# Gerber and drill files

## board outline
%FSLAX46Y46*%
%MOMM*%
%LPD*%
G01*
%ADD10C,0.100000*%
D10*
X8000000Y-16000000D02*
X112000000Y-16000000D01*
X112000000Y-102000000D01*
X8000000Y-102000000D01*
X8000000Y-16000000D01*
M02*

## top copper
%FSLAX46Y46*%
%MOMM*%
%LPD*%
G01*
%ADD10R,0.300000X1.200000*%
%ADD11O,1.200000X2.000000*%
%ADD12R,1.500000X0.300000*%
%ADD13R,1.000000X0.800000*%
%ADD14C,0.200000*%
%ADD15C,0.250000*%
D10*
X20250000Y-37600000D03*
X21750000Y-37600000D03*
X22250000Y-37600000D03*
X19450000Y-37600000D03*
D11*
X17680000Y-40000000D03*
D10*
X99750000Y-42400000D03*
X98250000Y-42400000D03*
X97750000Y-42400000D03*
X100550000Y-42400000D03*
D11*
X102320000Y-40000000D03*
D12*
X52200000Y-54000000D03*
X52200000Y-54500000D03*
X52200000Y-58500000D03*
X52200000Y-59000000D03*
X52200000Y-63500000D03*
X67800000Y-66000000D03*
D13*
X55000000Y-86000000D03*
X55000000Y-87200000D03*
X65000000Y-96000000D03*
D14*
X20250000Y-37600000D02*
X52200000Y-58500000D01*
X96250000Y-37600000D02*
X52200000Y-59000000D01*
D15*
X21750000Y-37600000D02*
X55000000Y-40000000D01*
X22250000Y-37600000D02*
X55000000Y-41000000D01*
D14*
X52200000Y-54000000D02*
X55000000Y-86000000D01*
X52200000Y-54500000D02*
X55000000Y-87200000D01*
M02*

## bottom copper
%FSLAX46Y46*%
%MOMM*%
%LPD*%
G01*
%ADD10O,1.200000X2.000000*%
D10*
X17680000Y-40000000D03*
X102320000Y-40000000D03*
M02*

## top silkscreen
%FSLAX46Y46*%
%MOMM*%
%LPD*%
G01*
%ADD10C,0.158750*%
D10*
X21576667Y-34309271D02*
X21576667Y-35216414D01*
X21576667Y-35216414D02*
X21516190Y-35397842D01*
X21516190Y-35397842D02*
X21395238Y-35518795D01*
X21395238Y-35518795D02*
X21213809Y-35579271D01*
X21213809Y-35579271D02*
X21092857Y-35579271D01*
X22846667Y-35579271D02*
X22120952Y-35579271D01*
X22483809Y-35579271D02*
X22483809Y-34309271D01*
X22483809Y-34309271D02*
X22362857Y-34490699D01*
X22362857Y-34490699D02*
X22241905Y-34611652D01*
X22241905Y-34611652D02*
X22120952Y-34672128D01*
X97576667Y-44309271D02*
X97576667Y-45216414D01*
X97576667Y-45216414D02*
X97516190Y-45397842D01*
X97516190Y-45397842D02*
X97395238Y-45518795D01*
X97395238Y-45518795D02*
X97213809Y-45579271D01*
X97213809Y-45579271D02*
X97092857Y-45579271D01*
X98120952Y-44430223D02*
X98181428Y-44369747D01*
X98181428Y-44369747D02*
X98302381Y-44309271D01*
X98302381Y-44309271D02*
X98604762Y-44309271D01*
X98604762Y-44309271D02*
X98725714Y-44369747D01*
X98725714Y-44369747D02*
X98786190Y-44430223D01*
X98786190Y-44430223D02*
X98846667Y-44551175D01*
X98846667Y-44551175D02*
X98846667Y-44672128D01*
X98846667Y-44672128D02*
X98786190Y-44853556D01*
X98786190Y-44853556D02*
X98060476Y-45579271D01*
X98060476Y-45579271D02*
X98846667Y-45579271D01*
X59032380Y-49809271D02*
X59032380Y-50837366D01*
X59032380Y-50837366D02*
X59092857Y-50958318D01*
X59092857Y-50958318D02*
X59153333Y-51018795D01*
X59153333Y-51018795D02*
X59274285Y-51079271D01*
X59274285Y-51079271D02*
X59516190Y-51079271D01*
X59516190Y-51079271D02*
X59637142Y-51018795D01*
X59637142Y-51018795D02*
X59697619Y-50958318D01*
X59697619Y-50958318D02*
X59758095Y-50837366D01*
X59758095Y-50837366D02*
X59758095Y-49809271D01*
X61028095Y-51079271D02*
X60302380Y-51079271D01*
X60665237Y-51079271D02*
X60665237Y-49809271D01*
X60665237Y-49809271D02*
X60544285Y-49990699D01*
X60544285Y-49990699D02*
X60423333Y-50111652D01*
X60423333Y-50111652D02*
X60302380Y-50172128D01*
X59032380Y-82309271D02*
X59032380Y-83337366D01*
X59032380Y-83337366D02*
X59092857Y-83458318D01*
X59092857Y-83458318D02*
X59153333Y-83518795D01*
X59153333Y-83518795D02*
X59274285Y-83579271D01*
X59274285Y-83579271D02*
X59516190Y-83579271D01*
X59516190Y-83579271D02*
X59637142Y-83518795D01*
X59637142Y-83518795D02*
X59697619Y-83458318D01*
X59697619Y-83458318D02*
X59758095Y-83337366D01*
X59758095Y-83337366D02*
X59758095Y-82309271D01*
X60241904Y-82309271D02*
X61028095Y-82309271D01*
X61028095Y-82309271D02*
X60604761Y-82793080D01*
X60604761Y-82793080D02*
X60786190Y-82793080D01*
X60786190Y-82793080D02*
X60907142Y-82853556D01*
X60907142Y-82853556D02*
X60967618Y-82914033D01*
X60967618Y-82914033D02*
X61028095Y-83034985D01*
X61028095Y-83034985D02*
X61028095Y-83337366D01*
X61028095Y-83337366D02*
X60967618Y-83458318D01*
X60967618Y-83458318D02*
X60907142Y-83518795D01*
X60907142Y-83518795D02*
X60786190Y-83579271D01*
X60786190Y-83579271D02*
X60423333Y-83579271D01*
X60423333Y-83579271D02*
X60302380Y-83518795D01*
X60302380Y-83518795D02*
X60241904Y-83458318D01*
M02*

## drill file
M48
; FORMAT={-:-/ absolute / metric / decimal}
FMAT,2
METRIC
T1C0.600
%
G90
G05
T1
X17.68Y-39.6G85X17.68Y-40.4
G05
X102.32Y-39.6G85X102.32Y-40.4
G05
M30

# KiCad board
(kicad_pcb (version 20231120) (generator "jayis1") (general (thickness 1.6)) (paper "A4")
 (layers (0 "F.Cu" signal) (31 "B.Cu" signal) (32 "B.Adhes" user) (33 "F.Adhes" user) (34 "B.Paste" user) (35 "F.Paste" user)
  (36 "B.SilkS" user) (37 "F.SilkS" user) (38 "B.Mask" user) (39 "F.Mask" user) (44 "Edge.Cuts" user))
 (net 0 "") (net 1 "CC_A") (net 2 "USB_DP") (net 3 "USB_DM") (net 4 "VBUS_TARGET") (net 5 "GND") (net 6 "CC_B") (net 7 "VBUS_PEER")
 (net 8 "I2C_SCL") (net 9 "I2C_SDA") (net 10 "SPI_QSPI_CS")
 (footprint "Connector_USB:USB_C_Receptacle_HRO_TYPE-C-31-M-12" (layer "F.Cu") (at 22 40)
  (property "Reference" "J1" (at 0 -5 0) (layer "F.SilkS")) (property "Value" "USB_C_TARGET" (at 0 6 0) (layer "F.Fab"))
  (pad "A5" smd rect (at -1.75 -2.4) (size 0.3 1.2) (layers "F.Cu" "F.Paste" "F.Mask") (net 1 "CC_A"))
  (pad "A6" smd rect (at -0.25 -2.4) (size 0.3 1.2) (layers "F.Cu" "F.Paste" "F.Mask") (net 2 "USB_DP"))
  (pad "A7" smd rect (at 0.25 -2.4) (size 0.3 1.2) (layers "F.Cu" "F.Paste" "F.Mask") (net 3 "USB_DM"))
  (pad "A4" smd rect (at -2.55 -2.4) (size 0.3 1.2) (layers "F.Cu" "F.Paste" "F.Mask") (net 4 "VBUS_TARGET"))
  (pad "S1" thru_hole oval (at -4.32 0) (size 1.2 2.0) (drill oval 0.6 1.4) (layers *.Cu *.Mask) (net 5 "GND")))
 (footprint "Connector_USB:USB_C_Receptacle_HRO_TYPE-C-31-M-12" (layer "F.Cu") (at 98 40 180)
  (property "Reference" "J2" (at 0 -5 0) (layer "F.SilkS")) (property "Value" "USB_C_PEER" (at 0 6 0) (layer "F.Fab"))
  (pad "A5" smd rect (at -1.75 -2.4) (size 0.3 1.2) (layers "F.Cu" "F.Paste" "F.Mask") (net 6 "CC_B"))
  (pad "A6" smd rect (at -0.25 -2.4) (size 0.3 1.2) (layers "F.Cu" "F.Paste" "F.Mask") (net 2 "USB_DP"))
  (pad "A7" smd rect (at 0.25 -2.4) (size 0.3 1.2) (layers "F.Cu" "F.Paste" "F.Mask") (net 3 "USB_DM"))
  (pad "A4" smd rect (at -2.55 -2.4) (size 0.3 1.2) (layers "F.Cu" "F.Paste" "F.Mask") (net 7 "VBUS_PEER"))
  (pad "S1" thru_hole oval (at -4.32 0) (size 1.2 2.0) (drill oval 0.6 1.4) (layers *.Cu *.Mask) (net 5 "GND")))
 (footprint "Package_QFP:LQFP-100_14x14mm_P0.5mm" (layer "F.Cu") (at 60 60) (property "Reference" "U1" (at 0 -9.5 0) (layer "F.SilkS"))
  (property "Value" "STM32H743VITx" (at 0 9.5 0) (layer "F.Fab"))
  (pad "1" smd rect (at -7.8 -6.0) (size 1.5 0.3) (layers "F.Cu" "F.Paste" "F.Mask") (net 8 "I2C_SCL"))
  (pad "2" smd rect (at -7.8 -5.5) (size 1.5 0.3) (layers "F.Cu" "F.Paste" "F.Mask") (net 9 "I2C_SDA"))
  (pad "10" smd rect (at -7.8 -1.5) (size 1.5 0.3) (layers "F.Cu" "F.Paste" "F.Mask") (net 1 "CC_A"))
  (pad "11" smd rect (at -7.8 -1.0) (size 1.5 0.3) (layers "F.Cu" "F.Paste" "F.Mask") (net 6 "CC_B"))
  (pad "20" smd rect (at -7.8 3.5) (size 1.5 0.3) (layers "F.Cu" "F.Paste" "F.Mask") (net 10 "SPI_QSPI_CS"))
  (pad "50" smd rect (at 7.8 6.0) (size 1.5 0.3) (layers "F.Cu" "F.Paste" "F.Mask") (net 5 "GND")))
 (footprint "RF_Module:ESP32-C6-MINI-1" (layer "F.Cu") (at 60 91) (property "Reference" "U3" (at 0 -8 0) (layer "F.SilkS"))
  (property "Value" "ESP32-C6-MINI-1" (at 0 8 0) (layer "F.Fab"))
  (pad "1" smd rect (at -5 -5) (size 1.0 0.8) (layers "F.Cu" "F.Paste" "F.Mask") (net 8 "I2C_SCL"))
  (pad "2" smd rect (at -5 -3.8) (size 1.0 0.8) (layers "F.Cu" "F.Paste" "F.Mask") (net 9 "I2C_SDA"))
  (pad "25" smd rect (at 5 5) (size 1.0 0.8) (layers "F.Cu" "F.Paste" "F.Mask") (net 5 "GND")))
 (segment (start 20.25 37.6) (end 52.2 58.5) (width 0.2) (layer "F.Cu") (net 1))
 (segment (start 96.25 37.6) (end 52.2 59.0) (width 0.2) (layer "F.Cu") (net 6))
 (segment (start 21.75 37.6) (end 55 40) (width 0.25) (layer "F.Cu") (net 2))
 (segment (start 22.25 37.6) (end 55 41) (width 0.25) (layer "F.Cu") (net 3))
 (segment (start 52.2 54.0) (end 55.0 86.0) (width 0.2) (layer "F.Cu") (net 8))
 (segment (start 52.2 54.5) (end 55.0 87.2) (width 0.2) (layer "F.Cu") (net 9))
 (gr_rect (start 8 16) (end 112 102) (stroke (width 0.1) (type default)) (fill none) (layer "Edge.Cuts")))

